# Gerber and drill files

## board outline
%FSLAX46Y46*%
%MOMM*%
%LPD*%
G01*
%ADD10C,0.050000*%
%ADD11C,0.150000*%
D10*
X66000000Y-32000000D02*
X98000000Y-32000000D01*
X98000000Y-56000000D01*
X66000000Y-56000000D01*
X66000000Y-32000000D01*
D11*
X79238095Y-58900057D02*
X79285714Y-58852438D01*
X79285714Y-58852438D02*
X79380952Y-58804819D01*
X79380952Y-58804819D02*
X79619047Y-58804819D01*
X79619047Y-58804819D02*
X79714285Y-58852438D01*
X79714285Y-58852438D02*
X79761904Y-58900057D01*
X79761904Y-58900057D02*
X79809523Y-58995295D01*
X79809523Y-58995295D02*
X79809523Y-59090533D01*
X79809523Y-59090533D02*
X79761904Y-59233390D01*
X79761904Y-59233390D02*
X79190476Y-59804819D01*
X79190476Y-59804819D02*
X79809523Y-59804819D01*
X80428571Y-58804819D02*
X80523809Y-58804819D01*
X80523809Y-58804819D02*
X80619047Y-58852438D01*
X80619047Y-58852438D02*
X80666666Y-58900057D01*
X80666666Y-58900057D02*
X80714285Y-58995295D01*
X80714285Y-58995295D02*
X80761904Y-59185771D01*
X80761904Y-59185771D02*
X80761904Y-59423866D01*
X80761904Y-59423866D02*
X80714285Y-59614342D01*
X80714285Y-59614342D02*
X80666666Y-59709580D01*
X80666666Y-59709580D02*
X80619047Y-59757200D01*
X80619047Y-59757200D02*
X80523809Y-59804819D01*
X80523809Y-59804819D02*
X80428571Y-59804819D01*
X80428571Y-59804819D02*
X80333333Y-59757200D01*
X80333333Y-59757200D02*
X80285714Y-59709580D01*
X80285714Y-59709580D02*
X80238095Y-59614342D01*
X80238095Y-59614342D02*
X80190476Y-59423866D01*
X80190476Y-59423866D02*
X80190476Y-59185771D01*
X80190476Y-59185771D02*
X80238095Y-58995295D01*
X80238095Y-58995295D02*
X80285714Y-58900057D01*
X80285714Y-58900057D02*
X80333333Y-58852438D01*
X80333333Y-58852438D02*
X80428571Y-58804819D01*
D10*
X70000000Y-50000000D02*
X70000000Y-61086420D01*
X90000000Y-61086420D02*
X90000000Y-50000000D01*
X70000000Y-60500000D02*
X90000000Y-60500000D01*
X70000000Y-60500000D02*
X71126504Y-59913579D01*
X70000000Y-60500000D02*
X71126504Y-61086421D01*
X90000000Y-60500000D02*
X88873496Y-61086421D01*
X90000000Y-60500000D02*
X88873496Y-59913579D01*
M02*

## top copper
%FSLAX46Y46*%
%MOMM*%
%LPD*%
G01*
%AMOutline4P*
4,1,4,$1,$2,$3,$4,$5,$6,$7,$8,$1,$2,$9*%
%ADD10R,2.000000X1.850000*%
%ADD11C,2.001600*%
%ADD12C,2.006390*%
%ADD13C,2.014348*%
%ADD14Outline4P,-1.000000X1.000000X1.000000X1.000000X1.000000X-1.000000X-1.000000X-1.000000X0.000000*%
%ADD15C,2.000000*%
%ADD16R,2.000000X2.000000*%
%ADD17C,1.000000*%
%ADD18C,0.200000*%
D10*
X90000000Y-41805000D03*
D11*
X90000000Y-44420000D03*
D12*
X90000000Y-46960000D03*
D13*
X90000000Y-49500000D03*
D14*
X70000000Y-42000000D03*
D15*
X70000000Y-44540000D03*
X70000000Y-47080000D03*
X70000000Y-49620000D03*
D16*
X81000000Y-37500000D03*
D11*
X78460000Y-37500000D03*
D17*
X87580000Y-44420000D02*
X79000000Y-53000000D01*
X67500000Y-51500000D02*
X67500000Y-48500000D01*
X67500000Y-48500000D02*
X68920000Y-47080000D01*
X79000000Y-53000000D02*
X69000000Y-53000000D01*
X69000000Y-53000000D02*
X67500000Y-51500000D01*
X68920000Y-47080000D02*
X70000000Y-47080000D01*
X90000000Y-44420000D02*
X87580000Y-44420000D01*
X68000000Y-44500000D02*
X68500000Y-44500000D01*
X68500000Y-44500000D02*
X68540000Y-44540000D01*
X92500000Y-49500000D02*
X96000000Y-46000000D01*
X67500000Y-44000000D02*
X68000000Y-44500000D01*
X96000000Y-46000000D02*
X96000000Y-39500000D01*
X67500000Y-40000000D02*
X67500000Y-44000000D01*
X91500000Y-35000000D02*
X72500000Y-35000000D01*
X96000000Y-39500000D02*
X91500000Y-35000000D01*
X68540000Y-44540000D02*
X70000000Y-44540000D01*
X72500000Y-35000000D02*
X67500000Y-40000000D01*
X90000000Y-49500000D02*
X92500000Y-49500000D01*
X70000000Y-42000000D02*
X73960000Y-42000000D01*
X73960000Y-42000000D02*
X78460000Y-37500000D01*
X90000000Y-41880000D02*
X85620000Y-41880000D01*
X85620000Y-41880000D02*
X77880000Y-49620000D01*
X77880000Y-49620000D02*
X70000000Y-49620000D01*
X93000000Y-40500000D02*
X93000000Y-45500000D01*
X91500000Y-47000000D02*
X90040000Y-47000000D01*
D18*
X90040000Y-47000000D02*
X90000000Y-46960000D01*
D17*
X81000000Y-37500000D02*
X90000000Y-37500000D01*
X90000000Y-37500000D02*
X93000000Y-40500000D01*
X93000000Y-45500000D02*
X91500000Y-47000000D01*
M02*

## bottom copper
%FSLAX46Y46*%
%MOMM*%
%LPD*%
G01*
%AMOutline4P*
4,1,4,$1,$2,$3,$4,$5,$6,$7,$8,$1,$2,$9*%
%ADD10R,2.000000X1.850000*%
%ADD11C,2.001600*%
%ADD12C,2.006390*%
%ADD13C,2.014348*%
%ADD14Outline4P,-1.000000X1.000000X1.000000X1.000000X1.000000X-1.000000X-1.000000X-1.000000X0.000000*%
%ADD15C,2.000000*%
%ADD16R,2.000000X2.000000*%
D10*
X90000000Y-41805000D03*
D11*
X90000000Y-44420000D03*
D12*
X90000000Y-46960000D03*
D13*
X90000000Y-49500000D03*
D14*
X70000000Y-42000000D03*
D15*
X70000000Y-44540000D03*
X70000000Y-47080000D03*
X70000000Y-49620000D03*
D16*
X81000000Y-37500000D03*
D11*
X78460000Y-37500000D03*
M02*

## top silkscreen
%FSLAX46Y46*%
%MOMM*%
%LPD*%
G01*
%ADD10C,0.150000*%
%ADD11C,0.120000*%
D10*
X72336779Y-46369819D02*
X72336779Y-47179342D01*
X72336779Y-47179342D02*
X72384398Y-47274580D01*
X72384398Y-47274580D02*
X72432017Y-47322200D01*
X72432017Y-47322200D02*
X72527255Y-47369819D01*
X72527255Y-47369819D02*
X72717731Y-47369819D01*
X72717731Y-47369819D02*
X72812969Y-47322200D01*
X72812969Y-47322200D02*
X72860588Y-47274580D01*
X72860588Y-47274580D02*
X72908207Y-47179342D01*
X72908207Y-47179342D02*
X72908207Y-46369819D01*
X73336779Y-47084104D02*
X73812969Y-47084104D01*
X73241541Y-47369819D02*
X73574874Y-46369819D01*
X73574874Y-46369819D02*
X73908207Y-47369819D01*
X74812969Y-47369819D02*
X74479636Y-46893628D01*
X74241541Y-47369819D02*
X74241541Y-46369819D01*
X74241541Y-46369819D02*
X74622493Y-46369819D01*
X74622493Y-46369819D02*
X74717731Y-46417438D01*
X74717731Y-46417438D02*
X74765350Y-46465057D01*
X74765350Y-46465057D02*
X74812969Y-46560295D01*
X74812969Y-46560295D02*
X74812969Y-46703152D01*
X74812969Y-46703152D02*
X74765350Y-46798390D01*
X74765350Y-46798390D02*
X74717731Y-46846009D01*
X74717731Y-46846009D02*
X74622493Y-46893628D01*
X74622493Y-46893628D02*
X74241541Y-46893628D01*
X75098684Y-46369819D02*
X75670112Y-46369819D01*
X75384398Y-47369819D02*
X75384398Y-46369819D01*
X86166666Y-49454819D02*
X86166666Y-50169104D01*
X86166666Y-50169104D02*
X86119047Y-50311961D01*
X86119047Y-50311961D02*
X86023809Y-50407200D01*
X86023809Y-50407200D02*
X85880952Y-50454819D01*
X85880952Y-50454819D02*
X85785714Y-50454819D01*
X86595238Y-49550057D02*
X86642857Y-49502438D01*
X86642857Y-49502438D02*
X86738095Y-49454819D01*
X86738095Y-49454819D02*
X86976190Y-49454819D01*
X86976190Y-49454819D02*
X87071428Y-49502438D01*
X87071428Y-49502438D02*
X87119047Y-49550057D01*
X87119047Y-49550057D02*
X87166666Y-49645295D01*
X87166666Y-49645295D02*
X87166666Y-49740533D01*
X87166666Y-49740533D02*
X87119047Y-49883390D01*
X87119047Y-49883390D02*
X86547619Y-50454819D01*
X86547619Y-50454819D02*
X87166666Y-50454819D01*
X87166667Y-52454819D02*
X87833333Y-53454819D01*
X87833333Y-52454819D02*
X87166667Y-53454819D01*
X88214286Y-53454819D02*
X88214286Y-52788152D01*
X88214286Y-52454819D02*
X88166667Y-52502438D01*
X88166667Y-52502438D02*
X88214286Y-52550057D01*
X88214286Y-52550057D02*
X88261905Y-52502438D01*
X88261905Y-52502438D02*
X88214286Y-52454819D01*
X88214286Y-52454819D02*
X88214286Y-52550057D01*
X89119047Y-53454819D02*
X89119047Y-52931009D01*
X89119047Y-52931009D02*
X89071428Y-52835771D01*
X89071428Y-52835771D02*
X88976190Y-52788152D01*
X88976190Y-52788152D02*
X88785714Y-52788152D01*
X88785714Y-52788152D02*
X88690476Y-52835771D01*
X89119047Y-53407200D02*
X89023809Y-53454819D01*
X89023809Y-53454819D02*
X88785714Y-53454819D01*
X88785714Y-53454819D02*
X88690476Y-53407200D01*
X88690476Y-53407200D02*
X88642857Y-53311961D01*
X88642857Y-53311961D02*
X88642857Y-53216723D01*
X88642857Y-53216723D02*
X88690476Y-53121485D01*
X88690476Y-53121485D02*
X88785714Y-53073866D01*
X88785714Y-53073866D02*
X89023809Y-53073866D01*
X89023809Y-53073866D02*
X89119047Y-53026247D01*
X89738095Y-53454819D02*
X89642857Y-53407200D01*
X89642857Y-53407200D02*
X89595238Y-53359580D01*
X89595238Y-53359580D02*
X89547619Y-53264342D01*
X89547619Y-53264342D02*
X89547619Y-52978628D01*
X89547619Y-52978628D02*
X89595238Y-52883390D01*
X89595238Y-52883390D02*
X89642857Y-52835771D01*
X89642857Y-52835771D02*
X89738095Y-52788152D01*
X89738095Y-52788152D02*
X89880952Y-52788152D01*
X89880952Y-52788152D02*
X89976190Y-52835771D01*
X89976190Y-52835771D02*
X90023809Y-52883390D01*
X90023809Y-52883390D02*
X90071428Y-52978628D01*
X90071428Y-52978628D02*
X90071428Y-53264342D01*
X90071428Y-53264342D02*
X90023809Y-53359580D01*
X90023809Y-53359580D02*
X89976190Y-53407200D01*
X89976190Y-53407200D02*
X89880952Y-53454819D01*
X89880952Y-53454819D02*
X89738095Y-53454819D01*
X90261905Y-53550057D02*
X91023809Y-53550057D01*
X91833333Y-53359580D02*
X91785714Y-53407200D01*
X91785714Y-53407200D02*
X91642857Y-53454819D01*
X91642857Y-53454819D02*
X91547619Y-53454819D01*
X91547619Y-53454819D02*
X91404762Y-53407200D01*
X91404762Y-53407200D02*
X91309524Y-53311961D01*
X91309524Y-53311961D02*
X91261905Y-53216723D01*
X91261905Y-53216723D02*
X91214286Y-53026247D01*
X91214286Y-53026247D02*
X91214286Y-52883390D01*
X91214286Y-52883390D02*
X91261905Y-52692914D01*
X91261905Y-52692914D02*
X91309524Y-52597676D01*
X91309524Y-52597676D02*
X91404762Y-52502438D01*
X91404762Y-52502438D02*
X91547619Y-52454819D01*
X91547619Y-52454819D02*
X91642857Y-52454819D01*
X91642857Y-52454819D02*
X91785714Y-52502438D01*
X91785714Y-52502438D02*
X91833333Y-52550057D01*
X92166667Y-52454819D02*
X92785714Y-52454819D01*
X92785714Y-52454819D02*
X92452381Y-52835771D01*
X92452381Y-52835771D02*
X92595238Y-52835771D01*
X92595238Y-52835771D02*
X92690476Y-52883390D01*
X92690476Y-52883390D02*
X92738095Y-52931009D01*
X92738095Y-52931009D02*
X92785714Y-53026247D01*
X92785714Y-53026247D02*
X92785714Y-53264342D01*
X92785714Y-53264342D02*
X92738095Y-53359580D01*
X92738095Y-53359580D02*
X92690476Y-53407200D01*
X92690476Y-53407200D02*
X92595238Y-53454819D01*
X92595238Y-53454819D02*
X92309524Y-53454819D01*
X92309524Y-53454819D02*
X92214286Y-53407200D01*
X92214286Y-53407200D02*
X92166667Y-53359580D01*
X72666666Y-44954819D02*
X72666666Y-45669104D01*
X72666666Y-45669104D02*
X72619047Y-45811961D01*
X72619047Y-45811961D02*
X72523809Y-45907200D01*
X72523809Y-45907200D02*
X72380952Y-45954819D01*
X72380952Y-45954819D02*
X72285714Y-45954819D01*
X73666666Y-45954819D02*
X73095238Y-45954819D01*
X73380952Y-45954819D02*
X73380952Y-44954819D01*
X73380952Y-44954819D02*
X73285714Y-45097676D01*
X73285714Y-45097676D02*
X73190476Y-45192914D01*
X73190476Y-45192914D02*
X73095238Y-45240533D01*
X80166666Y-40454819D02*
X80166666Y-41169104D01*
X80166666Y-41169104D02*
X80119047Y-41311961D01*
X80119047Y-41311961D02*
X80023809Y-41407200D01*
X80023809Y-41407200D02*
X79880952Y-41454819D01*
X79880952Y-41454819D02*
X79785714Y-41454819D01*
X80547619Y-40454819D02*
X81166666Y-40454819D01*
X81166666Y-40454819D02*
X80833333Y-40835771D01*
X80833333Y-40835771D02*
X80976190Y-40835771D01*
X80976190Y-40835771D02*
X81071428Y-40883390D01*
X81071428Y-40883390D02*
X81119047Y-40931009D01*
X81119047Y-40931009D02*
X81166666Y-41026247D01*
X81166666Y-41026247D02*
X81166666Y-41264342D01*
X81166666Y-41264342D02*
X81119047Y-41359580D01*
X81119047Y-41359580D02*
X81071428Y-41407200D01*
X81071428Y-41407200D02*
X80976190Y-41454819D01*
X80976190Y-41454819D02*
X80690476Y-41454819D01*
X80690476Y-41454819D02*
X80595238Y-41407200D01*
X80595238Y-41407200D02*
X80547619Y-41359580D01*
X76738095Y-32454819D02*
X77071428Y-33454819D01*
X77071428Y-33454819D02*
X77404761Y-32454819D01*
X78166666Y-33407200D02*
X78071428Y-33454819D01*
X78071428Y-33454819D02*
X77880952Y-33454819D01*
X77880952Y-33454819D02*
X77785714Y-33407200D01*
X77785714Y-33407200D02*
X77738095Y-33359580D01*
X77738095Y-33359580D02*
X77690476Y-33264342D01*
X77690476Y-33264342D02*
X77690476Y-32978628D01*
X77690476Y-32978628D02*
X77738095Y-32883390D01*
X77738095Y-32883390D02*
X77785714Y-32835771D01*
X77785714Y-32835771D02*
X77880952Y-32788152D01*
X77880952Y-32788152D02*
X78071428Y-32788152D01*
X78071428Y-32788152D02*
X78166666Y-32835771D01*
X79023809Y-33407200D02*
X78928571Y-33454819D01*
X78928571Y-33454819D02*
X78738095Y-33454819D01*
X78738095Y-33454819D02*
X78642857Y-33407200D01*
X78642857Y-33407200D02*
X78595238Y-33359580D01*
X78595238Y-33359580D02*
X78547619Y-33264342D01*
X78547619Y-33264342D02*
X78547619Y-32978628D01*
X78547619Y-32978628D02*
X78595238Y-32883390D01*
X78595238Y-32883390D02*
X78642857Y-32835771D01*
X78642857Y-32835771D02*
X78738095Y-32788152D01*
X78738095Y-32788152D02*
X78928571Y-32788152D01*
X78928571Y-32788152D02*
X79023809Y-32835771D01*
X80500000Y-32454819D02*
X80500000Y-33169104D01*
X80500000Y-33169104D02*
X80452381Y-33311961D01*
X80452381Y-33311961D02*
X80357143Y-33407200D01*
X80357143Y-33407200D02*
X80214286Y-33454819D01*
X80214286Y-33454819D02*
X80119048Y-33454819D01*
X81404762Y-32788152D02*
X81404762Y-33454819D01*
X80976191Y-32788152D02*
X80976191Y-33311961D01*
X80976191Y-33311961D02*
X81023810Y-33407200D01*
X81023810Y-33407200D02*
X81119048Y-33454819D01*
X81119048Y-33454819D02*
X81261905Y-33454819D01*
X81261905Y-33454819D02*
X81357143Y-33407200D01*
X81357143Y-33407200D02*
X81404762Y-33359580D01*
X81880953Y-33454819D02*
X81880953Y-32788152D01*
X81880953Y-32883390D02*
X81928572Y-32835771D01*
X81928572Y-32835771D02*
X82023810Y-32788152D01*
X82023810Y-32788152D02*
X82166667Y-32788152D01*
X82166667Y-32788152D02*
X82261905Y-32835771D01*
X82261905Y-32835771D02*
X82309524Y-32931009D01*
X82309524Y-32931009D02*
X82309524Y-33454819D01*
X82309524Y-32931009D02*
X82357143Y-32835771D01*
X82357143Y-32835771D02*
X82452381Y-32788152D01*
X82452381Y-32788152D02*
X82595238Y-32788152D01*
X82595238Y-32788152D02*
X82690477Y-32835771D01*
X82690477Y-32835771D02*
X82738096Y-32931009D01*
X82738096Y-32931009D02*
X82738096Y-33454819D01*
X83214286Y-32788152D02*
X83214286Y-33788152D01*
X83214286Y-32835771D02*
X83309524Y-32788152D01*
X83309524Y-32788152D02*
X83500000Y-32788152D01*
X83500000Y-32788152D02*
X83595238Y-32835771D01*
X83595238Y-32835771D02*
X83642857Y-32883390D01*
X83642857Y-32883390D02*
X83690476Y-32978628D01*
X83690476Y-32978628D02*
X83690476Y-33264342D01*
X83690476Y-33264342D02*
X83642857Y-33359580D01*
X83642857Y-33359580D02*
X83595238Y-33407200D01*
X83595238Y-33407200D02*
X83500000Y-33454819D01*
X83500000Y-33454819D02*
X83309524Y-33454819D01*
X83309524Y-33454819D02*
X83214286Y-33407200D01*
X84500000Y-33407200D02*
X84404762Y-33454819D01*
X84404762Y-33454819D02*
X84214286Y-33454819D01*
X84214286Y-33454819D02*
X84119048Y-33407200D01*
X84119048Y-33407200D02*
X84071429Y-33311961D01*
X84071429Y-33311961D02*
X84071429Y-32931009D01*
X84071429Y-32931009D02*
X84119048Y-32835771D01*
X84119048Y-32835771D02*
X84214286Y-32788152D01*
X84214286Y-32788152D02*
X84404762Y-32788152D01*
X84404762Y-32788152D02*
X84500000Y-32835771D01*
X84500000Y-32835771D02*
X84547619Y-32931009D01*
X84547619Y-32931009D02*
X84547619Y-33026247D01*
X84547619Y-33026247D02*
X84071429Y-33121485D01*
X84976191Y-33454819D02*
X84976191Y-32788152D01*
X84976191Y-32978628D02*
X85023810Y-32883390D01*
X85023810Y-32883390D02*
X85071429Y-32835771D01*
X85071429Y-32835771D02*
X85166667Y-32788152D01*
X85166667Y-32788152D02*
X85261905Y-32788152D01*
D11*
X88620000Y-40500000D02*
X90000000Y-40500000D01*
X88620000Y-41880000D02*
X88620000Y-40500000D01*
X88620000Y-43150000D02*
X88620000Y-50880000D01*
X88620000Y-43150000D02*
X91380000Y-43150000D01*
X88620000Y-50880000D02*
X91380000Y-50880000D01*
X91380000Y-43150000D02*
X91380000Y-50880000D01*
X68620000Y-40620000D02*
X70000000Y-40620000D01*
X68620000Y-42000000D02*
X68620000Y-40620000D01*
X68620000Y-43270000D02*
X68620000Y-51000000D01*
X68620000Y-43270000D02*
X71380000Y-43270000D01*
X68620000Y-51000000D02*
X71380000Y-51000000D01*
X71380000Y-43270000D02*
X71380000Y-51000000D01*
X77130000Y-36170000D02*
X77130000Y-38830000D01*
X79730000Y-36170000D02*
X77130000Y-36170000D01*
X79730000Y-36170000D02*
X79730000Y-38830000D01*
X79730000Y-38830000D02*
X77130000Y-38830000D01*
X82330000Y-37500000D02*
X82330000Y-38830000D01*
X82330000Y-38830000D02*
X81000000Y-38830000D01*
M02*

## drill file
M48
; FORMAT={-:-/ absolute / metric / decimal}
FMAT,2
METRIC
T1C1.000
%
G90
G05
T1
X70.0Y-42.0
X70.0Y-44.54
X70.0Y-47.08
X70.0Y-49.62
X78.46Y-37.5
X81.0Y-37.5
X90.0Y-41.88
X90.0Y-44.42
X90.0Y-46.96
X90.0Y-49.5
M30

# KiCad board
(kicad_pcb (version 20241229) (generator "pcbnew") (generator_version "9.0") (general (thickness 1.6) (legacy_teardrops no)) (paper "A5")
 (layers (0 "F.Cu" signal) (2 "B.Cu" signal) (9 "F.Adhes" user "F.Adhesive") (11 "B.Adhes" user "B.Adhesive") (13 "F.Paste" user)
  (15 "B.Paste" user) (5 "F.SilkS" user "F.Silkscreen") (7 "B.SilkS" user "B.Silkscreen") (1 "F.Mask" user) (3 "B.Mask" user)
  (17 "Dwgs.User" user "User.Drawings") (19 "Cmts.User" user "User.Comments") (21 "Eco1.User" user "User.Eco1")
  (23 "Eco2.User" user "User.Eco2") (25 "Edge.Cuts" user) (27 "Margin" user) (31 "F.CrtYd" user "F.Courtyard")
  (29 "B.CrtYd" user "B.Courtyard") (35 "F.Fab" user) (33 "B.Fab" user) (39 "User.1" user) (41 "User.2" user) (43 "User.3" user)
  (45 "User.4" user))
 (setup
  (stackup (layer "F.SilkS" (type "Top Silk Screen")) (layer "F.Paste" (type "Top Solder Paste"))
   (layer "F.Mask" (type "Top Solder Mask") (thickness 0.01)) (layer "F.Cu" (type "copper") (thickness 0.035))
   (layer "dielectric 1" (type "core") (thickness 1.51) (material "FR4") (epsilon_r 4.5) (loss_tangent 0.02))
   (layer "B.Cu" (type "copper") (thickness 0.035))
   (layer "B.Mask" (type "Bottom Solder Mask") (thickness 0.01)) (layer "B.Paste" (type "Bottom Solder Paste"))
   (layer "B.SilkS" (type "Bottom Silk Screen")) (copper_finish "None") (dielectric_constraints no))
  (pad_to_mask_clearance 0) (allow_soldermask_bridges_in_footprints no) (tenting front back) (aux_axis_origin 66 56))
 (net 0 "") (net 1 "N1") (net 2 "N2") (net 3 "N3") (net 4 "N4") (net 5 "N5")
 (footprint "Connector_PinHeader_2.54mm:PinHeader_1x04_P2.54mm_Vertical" (layer "F.Cu") (at 90 41.88)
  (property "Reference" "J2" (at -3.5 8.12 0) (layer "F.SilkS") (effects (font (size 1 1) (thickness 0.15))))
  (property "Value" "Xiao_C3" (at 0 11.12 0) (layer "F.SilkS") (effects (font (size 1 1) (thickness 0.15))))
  (fp_line (start -1.38 -1.38) (end 0 -1.38) (stroke (width 0.12) (type solid)) (layer "F.SilkS"))
  (fp_line (start -1.38 0) (end -1.38 -1.38) (stroke (width 0.12) (type solid)) (layer "F.SilkS"))
  (fp_line (start -1.38 1.27) (end -1.38 9) (stroke (width 0.12) (type solid)) (layer "F.SilkS"))
  (fp_line (start -1.38 1.27) (end 1.38 1.27) (stroke (width 0.12) (type solid)) (layer "F.SilkS"))
  (fp_line (start -1.38 9) (end 1.38 9) (stroke (width 0.12) (type solid)) (layer "F.SilkS"))
  (fp_line (start 1.38 1.27) (end 1.38 9) (stroke (width 0.12) (type solid)) (layer "F.SilkS"))
  (pad "1" thru_hole rect (at 0 0) (size 2 1.85) (drill 1 (offset 0 -0.075)) (layers "*.Cu" "*.Mask") (remove_unused_layers no) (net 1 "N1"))
  (pad "2" thru_hole circle (at 0 2.54) (size 2.0016 2.0016) (drill 1) (layers "*.Cu" "*.Mask") (remove_unused_layers no) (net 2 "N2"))
  (pad "3" thru_hole circle (at 0 5.08) (size 2.00639 2.00639) (drill 1) (layers "*.Cu" "*.Mask") (remove_unused_layers no) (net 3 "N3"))
  (pad "4" thru_hole circle (at 0 7.62) (size 2.014348 2.014348) (drill 1) (layers "*.Cu" "*.Mask") (remove_unused_layers no) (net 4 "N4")))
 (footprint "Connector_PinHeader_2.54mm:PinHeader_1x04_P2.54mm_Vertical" (layer "F.Cu") (at 70 42)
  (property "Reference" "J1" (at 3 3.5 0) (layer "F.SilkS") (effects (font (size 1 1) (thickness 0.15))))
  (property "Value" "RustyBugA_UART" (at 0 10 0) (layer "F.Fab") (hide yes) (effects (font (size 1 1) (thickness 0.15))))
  (fp_line (start -1.38 -1.38) (end 0 -1.38) (stroke (width 0.12) (type solid)) (layer "F.SilkS"))
  (fp_line (start -1.38 0) (end -1.38 -1.38) (stroke (width 0.12) (type solid)) (layer "F.SilkS"))
  (fp_line (start -1.38 1.27) (end -1.38 9) (stroke (width 0.12) (type solid)) (layer "F.SilkS"))
  (fp_line (start -1.38 1.27) (end 1.38 1.27) (stroke (width 0.12) (type solid)) (layer "F.SilkS"))
  (fp_line (start -1.38 9) (end 1.38 9) (stroke (width 0.12) (type solid)) (layer "F.SilkS"))
  (fp_line (start 1.38 1.27) (end 1.38 9) (stroke (width 0.12) (type solid)) (layer "F.SilkS"))
  (pad "1" thru_hole roundrect (at 0 0) (size 2 2) (drill 1) (layers "*.Cu" "*.Mask") (remove_unused_layers no) (roundrect_rratio 0)
   (chamfer_ratio 0.2) (chamfer) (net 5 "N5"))
  (pad "2" thru_hole circle (at 0 2.54) (size 2 2) (drill 1) (layers "*.Cu" "*.Mask") (remove_unused_layers no) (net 4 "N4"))
  (pad "3" thru_hole circle (at 0 5.08) (size 2 2) (drill 1) (layers "*.Cu" "*.Mask") (remove_unused_layers no) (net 2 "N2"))
  (pad "4" thru_hole circle (at 0 7.62) (size 2 2) (drill 1) (layers "*.Cu" "*.Mask") (remove_unused_layers no) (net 1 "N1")))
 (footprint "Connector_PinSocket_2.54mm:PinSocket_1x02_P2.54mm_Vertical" (layer "F.Cu") (at 81 37.5 -90)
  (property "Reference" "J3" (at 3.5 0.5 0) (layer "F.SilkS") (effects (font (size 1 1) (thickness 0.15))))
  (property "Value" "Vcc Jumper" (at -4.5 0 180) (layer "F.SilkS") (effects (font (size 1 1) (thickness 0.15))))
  (fp_line (start -1.33 3.87) (end 1.33 3.87) (stroke (width 0.12) (type solid)) (layer "F.SilkS"))
  (fp_line (start -1.33 1.27) (end -1.33 3.87) (stroke (width 0.12) (type solid)) (layer "F.SilkS"))
  (fp_line (start -1.33 1.27) (end 1.33 1.27) (stroke (width 0.12) (type solid)) (layer "F.SilkS"))
  (fp_line (start 1.33 1.27) (end 1.33 3.87) (stroke (width 0.12) (type solid)) (layer "F.SilkS"))
  (fp_line (start 0 -1.33) (end 1.33 -1.33) (stroke (width 0.12) (type solid)) (layer "F.SilkS"))
  (fp_line (start 1.33 -1.33) (end 1.33 0) (stroke (width 0.12) (type solid)) (layer "F.SilkS"))
  (pad "1" thru_hole rect (at 0 0 270) (size 2 2) (drill 1) (layers "*.Cu" "*.Mask") (remove_unused_layers no) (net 3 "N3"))
  (pad "2" thru_hole circle (at 0 2.54 270) (size 2.0016 2.0016) (drill 1) (layers "*.Cu" "*.Mask") (remove_unused_layers no) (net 5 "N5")))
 (gr_rect (start 66 32) (end 98 56) (stroke (width 0.05) (type default)) (fill no) (layer "Edge.Cuts"))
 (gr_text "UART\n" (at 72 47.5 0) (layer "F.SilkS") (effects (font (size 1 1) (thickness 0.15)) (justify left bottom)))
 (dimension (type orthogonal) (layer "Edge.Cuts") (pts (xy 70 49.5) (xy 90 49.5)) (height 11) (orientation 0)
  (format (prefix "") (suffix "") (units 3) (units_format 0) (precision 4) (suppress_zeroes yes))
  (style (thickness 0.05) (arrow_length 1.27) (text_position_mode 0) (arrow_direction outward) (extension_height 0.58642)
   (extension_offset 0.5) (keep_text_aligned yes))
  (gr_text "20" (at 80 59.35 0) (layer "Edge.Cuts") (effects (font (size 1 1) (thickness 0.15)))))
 (segment (start 87.58 44.42) (end 79 53) (width 1) (layer "F.Cu") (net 2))
 (segment (start 67.5 51.5) (end 67.5 48.5) (width 1) (layer "F.Cu") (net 2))
 (segment (start 67.5 48.5) (end 68.92 47.08) (width 1) (layer "F.Cu") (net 2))
 (segment (start 79 53) (end 69 53) (width 1) (layer "F.Cu") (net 2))
 (segment (start 69 53) (end 67.5 51.5) (width 1) (layer "F.Cu") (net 2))
 (segment (start 68.92 47.08) (end 70 47.08) (width 1) (layer "F.Cu") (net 2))
 (segment (start 90 44.42) (end 87.58 44.42) (width 1) (layer "F.Cu") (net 2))
 (segment (start 68 44.5) (end 68.5 44.5) (width 1) (layer "F.Cu") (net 4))
 (segment (start 68.5 44.5) (end 68.54 44.54) (width 1) (layer "F.Cu") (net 4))
 (segment (start 92.5 49.5) (end 96 46) (width 1) (layer "F.Cu") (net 4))
 (segment (start 67.5 44) (end 68 44.5) (width 1) (layer "F.Cu") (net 4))
 (segment (start 96 46) (end 96 39.5) (width 1) (layer "F.Cu") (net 4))
 (segment (start 67.5 40) (end 67.5 44) (width 1) (layer "F.Cu") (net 4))
 (segment (start 91.5 35) (end 72.5 35) (width 1) (layer "F.Cu") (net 4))
 (segment (start 96 39.5) (end 91.5 35) (width 1) (layer "F.Cu") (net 4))
 (segment (start 68.54 44.54) (end 70 44.54) (width 1) (layer "F.Cu") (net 4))
 (segment (start 72.5 35) (end 67.5 40) (width 1) (layer "F.Cu") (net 4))
 (segment (start 90 49.5) (end 92.5 49.5) (width 1) (layer "F.Cu") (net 4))
 (segment (start 70 42) (end 73.96 42) (width 1) (layer "F.Cu") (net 5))
 (segment (start 73.96 42) (end 78.46 37.5) (width 1) (layer "F.Cu") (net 5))
 (segment (start 90 41.88) (end 85.62 41.88) (width 1) (layer "F.Cu") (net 1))
 (segment (start 85.62 41.88) (end 77.88 49.62) (width 1) (layer "F.Cu") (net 1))
 (segment (start 77.88 49.62) (end 70 49.62) (width 1) (layer "F.Cu") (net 1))
 (segment (start 93 40.5) (end 93 45.5) (width 1) (layer "F.Cu") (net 3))
 (segment (start 91.5 47) (end 90.04 47) (width 1) (layer "F.Cu") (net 3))
 (segment (start 90.04 47) (end 90 46.96) (width 0.2) (layer "F.Cu") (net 3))
 (segment (start 81 37.5) (end 90 37.5) (width 1) (layer "F.Cu") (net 3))
 (segment (start 90 37.5) (end 93 40.5) (width 1) (layer "F.Cu") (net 3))
 (segment (start 93 45.5) (end 91.5 47) (width 1) (layer "F.Cu") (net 3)))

